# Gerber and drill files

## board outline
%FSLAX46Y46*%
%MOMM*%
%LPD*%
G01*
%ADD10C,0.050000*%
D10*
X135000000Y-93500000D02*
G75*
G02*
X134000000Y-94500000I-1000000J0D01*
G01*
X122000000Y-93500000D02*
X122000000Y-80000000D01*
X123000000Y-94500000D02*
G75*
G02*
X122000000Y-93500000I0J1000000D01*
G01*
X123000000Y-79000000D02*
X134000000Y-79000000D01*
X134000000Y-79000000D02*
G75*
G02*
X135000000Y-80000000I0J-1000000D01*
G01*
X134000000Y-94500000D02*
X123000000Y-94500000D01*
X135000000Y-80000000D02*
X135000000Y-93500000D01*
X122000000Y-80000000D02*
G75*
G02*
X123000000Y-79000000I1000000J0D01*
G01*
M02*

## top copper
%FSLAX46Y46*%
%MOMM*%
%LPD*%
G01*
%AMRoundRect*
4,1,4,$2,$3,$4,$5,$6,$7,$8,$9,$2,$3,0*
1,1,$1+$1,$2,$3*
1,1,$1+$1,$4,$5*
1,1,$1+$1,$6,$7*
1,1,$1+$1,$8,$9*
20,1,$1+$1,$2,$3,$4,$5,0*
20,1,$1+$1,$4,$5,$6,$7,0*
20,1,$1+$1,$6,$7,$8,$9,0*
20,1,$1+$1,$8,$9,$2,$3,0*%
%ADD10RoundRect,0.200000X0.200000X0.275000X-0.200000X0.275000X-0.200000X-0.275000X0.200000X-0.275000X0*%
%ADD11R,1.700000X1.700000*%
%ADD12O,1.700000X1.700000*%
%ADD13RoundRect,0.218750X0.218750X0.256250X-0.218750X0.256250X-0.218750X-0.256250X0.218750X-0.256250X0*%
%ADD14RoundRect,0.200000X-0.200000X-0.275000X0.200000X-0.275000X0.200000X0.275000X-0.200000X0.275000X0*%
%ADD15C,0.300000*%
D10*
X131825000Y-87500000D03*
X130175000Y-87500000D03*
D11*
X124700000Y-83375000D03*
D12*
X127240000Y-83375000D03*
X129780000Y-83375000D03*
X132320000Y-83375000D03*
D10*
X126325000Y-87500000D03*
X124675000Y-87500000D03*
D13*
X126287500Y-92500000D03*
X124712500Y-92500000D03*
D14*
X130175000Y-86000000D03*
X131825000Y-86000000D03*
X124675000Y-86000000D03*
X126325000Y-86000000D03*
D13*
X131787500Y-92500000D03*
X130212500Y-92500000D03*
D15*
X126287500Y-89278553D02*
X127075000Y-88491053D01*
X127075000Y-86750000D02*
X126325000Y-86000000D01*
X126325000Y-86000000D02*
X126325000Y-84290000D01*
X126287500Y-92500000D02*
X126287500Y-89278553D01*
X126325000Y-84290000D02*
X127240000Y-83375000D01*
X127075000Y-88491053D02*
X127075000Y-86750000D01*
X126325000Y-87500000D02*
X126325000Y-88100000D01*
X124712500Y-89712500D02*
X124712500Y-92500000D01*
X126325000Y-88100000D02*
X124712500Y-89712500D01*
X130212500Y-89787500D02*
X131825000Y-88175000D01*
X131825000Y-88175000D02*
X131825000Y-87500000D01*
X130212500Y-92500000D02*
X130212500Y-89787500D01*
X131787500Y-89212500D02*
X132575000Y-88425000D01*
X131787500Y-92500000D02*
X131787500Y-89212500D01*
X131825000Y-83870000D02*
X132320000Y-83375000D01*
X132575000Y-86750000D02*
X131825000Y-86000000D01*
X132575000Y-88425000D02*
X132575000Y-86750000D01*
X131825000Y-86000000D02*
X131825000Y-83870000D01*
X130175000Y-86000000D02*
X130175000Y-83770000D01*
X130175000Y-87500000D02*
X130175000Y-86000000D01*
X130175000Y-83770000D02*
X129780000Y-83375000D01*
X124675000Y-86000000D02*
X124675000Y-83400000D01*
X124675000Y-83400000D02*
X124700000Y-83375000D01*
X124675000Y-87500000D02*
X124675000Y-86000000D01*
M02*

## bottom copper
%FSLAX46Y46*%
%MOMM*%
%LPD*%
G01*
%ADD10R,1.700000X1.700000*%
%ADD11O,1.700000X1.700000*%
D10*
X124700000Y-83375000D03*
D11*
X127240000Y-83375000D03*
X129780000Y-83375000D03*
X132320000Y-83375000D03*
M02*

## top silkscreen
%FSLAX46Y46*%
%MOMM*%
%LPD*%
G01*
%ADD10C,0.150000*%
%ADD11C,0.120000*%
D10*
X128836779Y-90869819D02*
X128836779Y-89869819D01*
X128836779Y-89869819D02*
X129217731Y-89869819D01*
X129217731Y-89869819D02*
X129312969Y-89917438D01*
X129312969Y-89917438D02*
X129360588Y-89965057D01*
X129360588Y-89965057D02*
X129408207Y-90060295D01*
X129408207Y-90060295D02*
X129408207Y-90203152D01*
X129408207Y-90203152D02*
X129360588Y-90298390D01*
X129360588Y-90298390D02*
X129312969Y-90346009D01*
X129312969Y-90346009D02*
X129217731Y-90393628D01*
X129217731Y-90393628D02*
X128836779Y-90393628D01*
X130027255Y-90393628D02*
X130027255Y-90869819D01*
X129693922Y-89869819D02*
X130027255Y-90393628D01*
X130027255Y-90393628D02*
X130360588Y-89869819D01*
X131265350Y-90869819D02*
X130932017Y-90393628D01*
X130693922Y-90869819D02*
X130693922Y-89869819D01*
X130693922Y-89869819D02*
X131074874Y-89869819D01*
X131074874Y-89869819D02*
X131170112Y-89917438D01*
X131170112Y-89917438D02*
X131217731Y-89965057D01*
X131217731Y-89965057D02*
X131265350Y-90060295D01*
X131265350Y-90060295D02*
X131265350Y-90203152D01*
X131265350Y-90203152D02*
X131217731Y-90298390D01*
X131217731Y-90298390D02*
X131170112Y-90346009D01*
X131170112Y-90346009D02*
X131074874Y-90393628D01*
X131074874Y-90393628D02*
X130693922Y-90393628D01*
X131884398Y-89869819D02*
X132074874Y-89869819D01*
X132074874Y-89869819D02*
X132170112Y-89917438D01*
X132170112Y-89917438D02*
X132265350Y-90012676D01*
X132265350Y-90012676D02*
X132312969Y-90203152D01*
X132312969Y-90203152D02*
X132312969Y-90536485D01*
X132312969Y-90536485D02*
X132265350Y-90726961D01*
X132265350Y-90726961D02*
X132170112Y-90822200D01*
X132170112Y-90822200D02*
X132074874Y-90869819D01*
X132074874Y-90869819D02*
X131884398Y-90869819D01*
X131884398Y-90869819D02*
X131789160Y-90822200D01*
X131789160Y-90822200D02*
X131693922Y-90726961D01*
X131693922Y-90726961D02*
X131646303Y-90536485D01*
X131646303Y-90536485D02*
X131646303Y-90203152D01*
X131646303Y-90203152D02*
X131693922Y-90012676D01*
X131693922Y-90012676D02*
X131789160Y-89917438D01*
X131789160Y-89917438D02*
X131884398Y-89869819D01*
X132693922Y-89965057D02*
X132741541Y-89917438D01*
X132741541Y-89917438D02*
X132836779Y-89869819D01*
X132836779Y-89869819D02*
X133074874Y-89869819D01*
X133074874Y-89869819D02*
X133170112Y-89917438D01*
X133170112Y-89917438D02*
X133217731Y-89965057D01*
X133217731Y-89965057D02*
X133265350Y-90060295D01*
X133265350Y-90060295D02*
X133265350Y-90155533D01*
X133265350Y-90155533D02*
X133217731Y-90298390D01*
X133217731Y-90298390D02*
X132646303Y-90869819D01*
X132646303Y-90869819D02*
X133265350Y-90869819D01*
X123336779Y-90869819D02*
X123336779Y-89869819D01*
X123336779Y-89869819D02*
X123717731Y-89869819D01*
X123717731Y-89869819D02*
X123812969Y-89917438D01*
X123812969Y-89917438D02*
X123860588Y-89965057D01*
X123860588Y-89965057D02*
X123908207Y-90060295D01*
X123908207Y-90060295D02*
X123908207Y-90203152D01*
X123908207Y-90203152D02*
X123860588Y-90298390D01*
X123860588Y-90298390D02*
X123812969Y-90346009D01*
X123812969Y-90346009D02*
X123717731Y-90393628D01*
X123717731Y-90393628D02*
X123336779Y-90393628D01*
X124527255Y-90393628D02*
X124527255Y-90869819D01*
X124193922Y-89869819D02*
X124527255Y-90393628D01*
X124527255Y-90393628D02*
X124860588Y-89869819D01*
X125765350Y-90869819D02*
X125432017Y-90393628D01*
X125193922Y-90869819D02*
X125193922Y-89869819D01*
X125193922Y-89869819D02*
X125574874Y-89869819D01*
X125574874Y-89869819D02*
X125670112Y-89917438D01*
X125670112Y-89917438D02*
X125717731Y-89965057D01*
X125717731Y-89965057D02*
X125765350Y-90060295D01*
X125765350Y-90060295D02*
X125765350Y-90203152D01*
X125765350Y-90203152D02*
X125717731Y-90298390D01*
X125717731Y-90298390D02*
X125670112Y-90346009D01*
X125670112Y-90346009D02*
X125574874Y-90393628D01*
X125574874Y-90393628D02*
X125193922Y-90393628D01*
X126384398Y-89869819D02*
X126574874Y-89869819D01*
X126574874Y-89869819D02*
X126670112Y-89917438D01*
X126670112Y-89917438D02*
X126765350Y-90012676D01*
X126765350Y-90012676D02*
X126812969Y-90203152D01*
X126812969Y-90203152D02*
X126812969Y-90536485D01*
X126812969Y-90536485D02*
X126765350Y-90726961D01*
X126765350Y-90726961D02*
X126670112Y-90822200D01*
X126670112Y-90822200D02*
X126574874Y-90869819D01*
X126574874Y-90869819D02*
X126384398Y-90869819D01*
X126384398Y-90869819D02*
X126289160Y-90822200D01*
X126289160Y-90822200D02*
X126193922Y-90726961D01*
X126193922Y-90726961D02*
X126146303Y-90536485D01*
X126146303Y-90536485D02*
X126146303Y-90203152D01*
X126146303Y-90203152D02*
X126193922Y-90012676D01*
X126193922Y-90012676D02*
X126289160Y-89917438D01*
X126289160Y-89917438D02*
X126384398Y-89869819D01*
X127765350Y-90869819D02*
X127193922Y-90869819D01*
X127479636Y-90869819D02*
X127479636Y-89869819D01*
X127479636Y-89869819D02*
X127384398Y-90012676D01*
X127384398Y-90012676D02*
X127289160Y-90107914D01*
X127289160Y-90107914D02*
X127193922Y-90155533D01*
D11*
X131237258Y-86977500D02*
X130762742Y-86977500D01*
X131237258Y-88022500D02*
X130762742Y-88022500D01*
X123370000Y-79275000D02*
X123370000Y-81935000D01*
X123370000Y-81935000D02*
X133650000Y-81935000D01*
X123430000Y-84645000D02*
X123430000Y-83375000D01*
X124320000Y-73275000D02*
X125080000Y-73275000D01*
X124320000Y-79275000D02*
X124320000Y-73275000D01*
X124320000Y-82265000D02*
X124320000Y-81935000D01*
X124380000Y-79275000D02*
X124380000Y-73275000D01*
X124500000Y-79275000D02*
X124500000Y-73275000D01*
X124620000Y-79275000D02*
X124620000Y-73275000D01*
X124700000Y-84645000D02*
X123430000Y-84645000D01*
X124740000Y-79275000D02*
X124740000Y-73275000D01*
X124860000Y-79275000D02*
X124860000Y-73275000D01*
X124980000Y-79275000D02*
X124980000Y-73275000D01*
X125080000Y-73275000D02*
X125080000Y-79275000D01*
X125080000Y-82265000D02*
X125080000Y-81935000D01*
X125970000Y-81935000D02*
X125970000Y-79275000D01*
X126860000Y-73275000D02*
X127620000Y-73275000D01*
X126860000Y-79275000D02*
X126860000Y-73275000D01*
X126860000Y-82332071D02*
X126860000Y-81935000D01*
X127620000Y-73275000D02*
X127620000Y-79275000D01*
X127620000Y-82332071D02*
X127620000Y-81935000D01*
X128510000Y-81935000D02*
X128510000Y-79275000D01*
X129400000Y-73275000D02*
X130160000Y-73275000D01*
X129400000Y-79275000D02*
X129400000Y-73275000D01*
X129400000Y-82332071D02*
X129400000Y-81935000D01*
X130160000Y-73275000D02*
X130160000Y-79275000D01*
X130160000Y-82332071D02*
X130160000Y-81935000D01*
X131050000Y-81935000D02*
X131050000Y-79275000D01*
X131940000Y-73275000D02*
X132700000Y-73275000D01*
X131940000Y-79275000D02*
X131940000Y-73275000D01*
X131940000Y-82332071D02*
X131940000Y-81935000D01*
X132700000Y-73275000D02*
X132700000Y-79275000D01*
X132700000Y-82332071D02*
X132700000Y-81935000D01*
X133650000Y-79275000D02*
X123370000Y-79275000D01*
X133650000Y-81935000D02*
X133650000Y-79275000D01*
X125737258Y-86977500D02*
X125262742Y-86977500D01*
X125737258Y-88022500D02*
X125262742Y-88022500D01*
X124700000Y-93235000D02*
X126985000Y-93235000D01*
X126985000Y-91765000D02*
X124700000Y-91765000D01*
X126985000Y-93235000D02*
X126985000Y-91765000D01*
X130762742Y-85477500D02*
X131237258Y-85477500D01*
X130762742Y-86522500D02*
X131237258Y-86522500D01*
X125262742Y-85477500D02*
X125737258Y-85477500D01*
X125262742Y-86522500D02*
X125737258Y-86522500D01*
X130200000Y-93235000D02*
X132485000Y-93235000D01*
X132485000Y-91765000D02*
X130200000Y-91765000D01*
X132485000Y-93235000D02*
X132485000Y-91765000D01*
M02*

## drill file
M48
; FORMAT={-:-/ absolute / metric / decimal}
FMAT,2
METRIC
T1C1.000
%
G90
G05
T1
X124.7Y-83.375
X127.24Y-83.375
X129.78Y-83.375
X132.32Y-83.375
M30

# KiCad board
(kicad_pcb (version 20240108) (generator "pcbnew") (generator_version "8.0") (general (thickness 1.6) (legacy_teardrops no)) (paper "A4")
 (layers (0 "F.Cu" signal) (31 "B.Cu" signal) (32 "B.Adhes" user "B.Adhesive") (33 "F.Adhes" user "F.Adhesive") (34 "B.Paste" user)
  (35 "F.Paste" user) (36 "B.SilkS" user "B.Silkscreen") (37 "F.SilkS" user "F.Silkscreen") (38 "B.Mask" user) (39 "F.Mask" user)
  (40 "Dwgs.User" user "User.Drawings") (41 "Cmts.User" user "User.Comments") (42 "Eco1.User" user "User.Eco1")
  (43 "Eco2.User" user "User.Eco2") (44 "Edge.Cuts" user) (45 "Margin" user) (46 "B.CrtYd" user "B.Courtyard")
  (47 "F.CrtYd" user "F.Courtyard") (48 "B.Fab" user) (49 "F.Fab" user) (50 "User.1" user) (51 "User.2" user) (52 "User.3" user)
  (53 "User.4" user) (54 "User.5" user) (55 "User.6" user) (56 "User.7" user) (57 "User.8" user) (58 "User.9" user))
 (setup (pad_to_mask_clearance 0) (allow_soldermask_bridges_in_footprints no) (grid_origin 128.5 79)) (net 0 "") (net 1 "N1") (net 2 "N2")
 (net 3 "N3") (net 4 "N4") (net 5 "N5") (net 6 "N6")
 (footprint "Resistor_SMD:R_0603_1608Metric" (layer "F.Cu") (at 131 87.5 180)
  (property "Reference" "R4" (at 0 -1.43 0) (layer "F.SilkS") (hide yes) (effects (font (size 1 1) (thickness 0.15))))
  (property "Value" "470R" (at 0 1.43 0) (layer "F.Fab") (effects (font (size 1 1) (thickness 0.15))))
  (fp_line (start -0.237258 0.5225) (end 0.237258 0.5225) (stroke (width 0.12) (type solid)) (layer "F.SilkS"))
  (fp_line (start -0.237258 -0.5225) (end 0.237258 -0.5225) (stroke (width 0.12) (type solid)) (layer "F.SilkS"))
  (pad "1" smd roundrect (at -0.825 0 180) (size 0.8 0.95) (layers "F.Cu" "F.Paste" "F.Mask") (roundrect_rratio 0.25) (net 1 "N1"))
  (pad "2" smd roundrect (at 0.825 0 180) (size 0.8 0.95) (layers "F.Cu" "F.Paste" "F.Mask") (roundrect_rratio 0.25) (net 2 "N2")))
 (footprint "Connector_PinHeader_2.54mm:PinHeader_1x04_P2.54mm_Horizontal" (layer "F.Cu") (at 124.7 83.375 90)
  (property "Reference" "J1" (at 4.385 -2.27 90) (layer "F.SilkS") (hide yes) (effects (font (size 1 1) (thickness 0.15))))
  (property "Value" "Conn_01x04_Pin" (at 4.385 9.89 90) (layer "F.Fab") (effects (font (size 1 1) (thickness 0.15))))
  (fp_line (start 4.1 -1.33) (end 1.44 -1.33) (stroke (width 0.12) (type solid)) (layer "F.SilkS"))
  (fp_line (start 1.44 -1.33) (end 1.44 8.95) (stroke (width 0.12) (type solid)) (layer "F.SilkS"))
  (fp_line (start -1.27 -1.27) (end 0 -1.27) (stroke (width 0.12) (type solid)) (layer "F.SilkS"))
  (fp_line (start 10.1 -0.38) (end 10.1 0.38) (stroke (width 0.12) (type solid)) (layer "F.SilkS"))
  (fp_line (start 4.1 -0.38) (end 10.1 -0.38) (stroke (width 0.12) (type solid)) (layer "F.SilkS"))
  (fp_line (start 1.11 -0.38) (end 1.44 -0.38) (stroke (width 0.12) (type solid)) (layer "F.SilkS"))
  (fp_line (start 4.1 -0.32) (end 10.1 -0.32) (stroke (width 0.12) (type solid)) (layer "F.SilkS"))
  (fp_line (start 4.1 -0.2) (end 10.1 -0.2) (stroke (width 0.12) (type solid)) (layer "F.SilkS"))
  (fp_line (start 4.1 -0.08) (end 10.1 -0.08) (stroke (width 0.12) (type solid)) (layer "F.SilkS"))
  (fp_line (start -1.27 0) (end -1.27 -1.27) (stroke (width 0.12) (type solid)) (layer "F.SilkS"))
  (fp_line (start 4.1 0.04) (end 10.1 0.04) (stroke (width 0.12) (type solid)) (layer "F.SilkS"))
  (fp_line (start 4.1 0.16) (end 10.1 0.16) (stroke (width 0.12) (type solid)) (layer "F.SilkS"))
  (fp_line (start 4.1 0.28) (end 10.1 0.28) (stroke (width 0.12) (type solid)) (layer "F.SilkS"))
  (fp_line (start 10.1 0.38) (end 4.1 0.38) (stroke (width 0.12) (type solid)) (layer "F.SilkS"))
  (fp_line (start 1.11 0.38) (end 1.44 0.38) (stroke (width 0.12) (type solid)) (layer "F.SilkS"))
  (fp_line (start 1.44 1.27) (end 4.1 1.27) (stroke (width 0.12) (type solid)) (layer "F.SilkS"))
  (fp_line (start 10.1 2.16) (end 10.1 2.92) (stroke (width 0.12) (type solid)) (layer "F.SilkS"))
  (fp_line (start 4.1 2.16) (end 10.1 2.16) (stroke (width 0.12) (type solid)) (layer "F.SilkS"))
  (fp_line (start 1.042929 2.16) (end 1.44 2.16) (stroke (width 0.12) (type solid)) (layer "F.SilkS"))
  (fp_line (start 10.1 2.92) (end 4.1 2.92) (stroke (width 0.12) (type solid)) (layer "F.SilkS"))
  (fp_line (start 1.042929 2.92) (end 1.44 2.92) (stroke (width 0.12) (type solid)) (layer "F.SilkS"))
  (fp_line (start 1.44 3.81) (end 4.1 3.81) (stroke (width 0.12) (type solid)) (layer "F.SilkS"))
  (fp_line (start 10.1 4.7) (end 10.1 5.46) (stroke (width 0.12) (type solid)) (layer "F.SilkS"))
  (fp_line (start 4.1 4.7) (end 10.1 4.7) (stroke (width 0.12) (type solid)) (layer "F.SilkS"))
  (fp_line (start 1.042929 4.7) (end 1.44 4.7) (stroke (width 0.12) (type solid)) (layer "F.SilkS"))
  (fp_line (start 10.1 5.46) (end 4.1 5.46) (stroke (width 0.12) (type solid)) (layer "F.SilkS"))
  (fp_line (start 1.042929 5.46) (end 1.44 5.46) (stroke (width 0.12) (type solid)) (layer "F.SilkS"))
  (fp_line (start 1.44 6.35) (end 4.1 6.35) (stroke (width 0.12) (type solid)) (layer "F.SilkS"))
  (fp_line (start 10.1 7.24) (end 10.1 8) (stroke (width 0.12) (type solid)) (layer "F.SilkS"))
  (fp_line (start 4.1 7.24) (end 10.1 7.24) (stroke (width 0.12) (type solid)) (layer "F.SilkS"))
  (fp_line (start 1.042929 7.24) (end 1.44 7.24) (stroke (width 0.12) (type solid)) (layer "F.SilkS"))
  (fp_line (start 10.1 8) (end 4.1 8) (stroke (width 0.12) (type solid)) (layer "F.SilkS"))
  (fp_line (start 1.042929 8) (end 1.44 8) (stroke (width 0.12) (type solid)) (layer "F.SilkS"))
  (fp_line (start 4.1 8.95) (end 4.1 -1.33) (stroke (width 0.12) (type solid)) (layer "F.SilkS"))
  (fp_line (start 1.44 8.95) (end 4.1 8.95) (stroke (width 0.12) (type solid)) (layer "F.SilkS"))
  (pad "1" thru_hole rect (at 0 0 90) (size 1.7 1.7) (drill 1) (layers "*.Cu" "*.Mask") (remove_unused_layers no) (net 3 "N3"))
  (pad "2" thru_hole oval (at 0 2.54 90) (size 1.7 1.7) (drill 1) (layers "*.Cu" "*.Mask") (remove_unused_layers no) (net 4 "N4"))
  (pad "3" thru_hole oval (at 0 5.08 90) (size 1.7 1.7) (drill 1) (layers "*.Cu" "*.Mask") (remove_unused_layers no) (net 2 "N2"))
  (pad "4" thru_hole oval (at 0 7.62 90) (size 1.7 1.7) (drill 1) (layers "*.Cu" "*.Mask") (remove_unused_layers no) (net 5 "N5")))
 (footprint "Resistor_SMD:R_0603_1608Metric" (layer "F.Cu") (at 125.5 87.5 180)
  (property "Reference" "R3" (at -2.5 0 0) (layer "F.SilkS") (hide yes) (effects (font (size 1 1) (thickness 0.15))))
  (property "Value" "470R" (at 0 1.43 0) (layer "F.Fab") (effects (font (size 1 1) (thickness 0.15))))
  (fp_line (start -0.237258 0.5225) (end 0.237258 0.5225) (stroke (width 0.12) (type solid)) (layer "F.SilkS"))
  (fp_line (start -0.237258 -0.5225) (end 0.237258 -0.5225) (stroke (width 0.12) (type solid)) (layer "F.SilkS"))
  (pad "1" smd roundrect (at -0.825 0 180) (size 0.8 0.95) (layers "F.Cu" "F.Paste" "F.Mask") (roundrect_rratio 0.25) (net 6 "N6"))
  (pad "2" smd roundrect (at 0.825 0 180) (size 0.8 0.95) (layers "F.Cu" "F.Paste" "F.Mask") (roundrect_rratio 0.25) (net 3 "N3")))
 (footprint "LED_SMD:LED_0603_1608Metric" (layer "F.Cu") (at 125.5 92.5 180)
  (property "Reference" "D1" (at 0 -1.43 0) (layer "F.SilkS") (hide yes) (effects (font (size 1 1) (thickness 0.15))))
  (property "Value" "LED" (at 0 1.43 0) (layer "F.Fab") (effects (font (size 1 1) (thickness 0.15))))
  (fp_line (start 0.8 -0.735) (end -1.485 -0.735) (stroke (width 0.12) (type solid)) (layer "F.SilkS"))
  (fp_line (start -1.485 0.735) (end 0.8 0.735) (stroke (width 0.12) (type solid)) (layer "F.SilkS"))
  (fp_line (start -1.485 -0.735) (end -1.485 0.735) (stroke (width 0.12) (type solid)) (layer "F.SilkS"))
  (pad "1" smd roundrect (at -0.7875 0 180) (size 0.875 0.95) (layers "F.Cu" "F.Paste" "F.Mask") (roundrect_rratio 0.25) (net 4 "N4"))
  (pad "2" smd roundrect (at 0.7875 0 180) (size 0.875 0.95) (layers "F.Cu" "F.Paste" "F.Mask") (roundrect_rratio 0.25) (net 6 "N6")))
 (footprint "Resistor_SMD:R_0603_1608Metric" (layer "F.Cu") (at 131 86)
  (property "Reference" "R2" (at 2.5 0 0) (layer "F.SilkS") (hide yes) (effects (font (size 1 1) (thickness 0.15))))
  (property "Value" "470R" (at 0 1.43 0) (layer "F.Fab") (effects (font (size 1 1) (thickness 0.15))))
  (fp_line (start -0.237258 -0.5225) (end 0.237258 -0.5225) (stroke (width 0.12) (type solid)) (layer "F.SilkS"))
  (fp_line (start -0.237258 0.5225) (end 0.237258 0.5225) (stroke (width 0.12) (type solid)) (layer "F.SilkS"))
  (pad "1" smd roundrect (at -0.825 0) (size 0.8 0.95) (layers "F.Cu" "F.Paste" "F.Mask") (roundrect_rratio 0.25) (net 2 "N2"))
  (pad "2" smd roundrect (at 0.825 0) (size 0.8 0.95) (layers "F.Cu" "F.Paste" "F.Mask") (roundrect_rratio 0.25) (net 5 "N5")))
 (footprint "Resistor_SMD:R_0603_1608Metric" (layer "F.Cu") (at 125.5 86)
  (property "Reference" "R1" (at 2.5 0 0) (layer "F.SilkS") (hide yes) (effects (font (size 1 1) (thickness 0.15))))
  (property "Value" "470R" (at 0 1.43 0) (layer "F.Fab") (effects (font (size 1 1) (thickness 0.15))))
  (fp_line (start -0.237258 -0.5225) (end 0.237258 -0.5225) (stroke (width 0.12) (type solid)) (layer "F.SilkS"))
  (fp_line (start -0.237258 0.5225) (end 0.237258 0.5225) (stroke (width 0.12) (type solid)) (layer "F.SilkS"))
  (pad "1" smd roundrect (at -0.825 0) (size 0.8 0.95) (layers "F.Cu" "F.Paste" "F.Mask") (roundrect_rratio 0.25) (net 3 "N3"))
  (pad "2" smd roundrect (at 0.825 0) (size 0.8 0.95) (layers "F.Cu" "F.Paste" "F.Mask") (roundrect_rratio 0.25) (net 4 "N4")))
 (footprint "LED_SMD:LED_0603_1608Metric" (layer "F.Cu") (at 131 92.5 180)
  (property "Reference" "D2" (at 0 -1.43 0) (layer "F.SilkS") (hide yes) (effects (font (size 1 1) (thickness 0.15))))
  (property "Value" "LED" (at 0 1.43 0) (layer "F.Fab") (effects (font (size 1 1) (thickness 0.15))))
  (fp_line (start 0.8 -0.735) (end -1.485 -0.735) (stroke (width 0.12) (type solid)) (layer "F.SilkS"))
  (fp_line (start -1.485 0.735) (end 0.8 0.735) (stroke (width 0.12) (type solid)) (layer "F.SilkS"))
  (fp_line (start -1.485 -0.735) (end -1.485 0.735) (stroke (width 0.12) (type solid)) (layer "F.SilkS"))
  (pad "1" smd roundrect (at -0.7875 0 180) (size 0.875 0.95) (layers "F.Cu" "F.Paste" "F.Mask") (roundrect_rratio 0.25) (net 5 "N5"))
  (pad "2" smd roundrect (at 0.7875 0 180) (size 0.875 0.95) (layers "F.Cu" "F.Paste" "F.Mask") (roundrect_rratio 0.25) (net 1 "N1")))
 (gr_arc (start 135 93.5) (mid 134.707107 94.207107) (end 134 94.5) (stroke (width 0.05) (type default)) (layer "Edge.Cuts"))
 (gr_line (start 122 93.5) (end 122 80) (stroke (width 0.05) (type default)) (layer "Edge.Cuts"))
 (gr_arc (start 123 94.5) (mid 122.292893 94.207107) (end 122 93.5) (stroke (width 0.05) (type default)) (layer "Edge.Cuts"))
 (gr_line (start 123 79) (end 134 79) (stroke (width 0.05) (type default)) (layer "Edge.Cuts"))
 (gr_arc (start 134 79) (mid 134.707107 79.292893) (end 135 80) (stroke (width 0.05) (type default)) (layer "Edge.Cuts"))
 (gr_line (start 134 94.5) (end 123 94.5) (stroke (width 0.05) (type default)) (layer "Edge.Cuts"))
 (gr_line (start 135 80) (end 135 93.5) (stroke (width 0.05) (type default)) (layer "Edge.Cuts"))
 (gr_arc (start 122 80) (mid 122.292893 79.292893) (end 123 79) (stroke (width 0.05) (type default)) (layer "Edge.Cuts"))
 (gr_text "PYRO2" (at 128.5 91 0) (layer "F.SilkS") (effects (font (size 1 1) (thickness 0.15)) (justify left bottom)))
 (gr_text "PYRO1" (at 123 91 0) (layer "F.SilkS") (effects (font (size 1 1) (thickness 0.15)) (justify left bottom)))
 (segment (start 126.2875 89.278553) (end 127.075 88.491053) (width 0.3) (layer "F.Cu") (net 4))
 (segment (start 127.075 86.75) (end 126.325 86) (width 0.3) (layer "F.Cu") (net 4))
 (segment (start 126.325 86) (end 126.325 84.29) (width 0.3) (layer "F.Cu") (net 4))
 (segment (start 126.2875 92.5) (end 126.2875 89.278553) (width 0.3) (layer "F.Cu") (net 4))
 (segment (start 126.325 84.29) (end 127.24 83.375) (width 0.3) (layer "F.Cu") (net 4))
 (segment (start 127.075 88.491053) (end 127.075 86.75) (width 0.3) (layer "F.Cu") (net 4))
 (segment (start 126.325 87.5) (end 126.325 88.1) (width 0.3) (layer "F.Cu") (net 6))
 (segment (start 124.7125 89.7125) (end 124.7125 92.5) (width 0.3) (layer "F.Cu") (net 6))
 (segment (start 126.325 88.1) (end 124.7125 89.7125) (width 0.3) (layer "F.Cu") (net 6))
 (segment (start 130.2125 89.7875) (end 131.825 88.175) (width 0.3) (layer "F.Cu") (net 1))
 (segment (start 131.825 88.175) (end 131.825 87.5) (width 0.3) (layer "F.Cu") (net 1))
 (segment (start 130.2125 92.5) (end 130.2125 89.7875) (width 0.3) (layer "F.Cu") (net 1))
 (segment (start 131.7875 89.2125) (end 132.575 88.425) (width 0.3) (layer "F.Cu") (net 5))
 (segment (start 131.7875 92.5) (end 131.7875 89.2125) (width 0.3) (layer "F.Cu") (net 5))
 (segment (start 131.825 83.87) (end 132.32 83.375) (width 0.3) (layer "F.Cu") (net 5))
 (segment (start 132.575 86.75) (end 131.825 86) (width 0.3) (layer "F.Cu") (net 5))
 (segment (start 132.575 88.425) (end 132.575 86.75) (width 0.3) (layer "F.Cu") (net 5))
 (segment (start 131.825 86) (end 131.825 83.87) (width 0.3) (layer "F.Cu") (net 5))
 (segment (start 130.175 86) (end 130.175 83.77) (width 0.3) (layer "F.Cu") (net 2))
 (segment (start 130.175 87.5) (end 130.175 86) (width 0.3) (layer "F.Cu") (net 2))
 (segment (start 130.175 83.77) (end 129.78 83.375) (width 0.3) (layer "F.Cu") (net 2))
 (segment (start 124.675 86) (end 124.675 83.4) (width 0.3) (layer "F.Cu") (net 3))
 (segment (start 124.675 83.4) (end 124.7 83.375) (width 0.3) (layer "F.Cu") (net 3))
 (segment (start 124.675 87.5) (end 124.675 86) (width 0.3) (layer "F.Cu") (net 3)))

